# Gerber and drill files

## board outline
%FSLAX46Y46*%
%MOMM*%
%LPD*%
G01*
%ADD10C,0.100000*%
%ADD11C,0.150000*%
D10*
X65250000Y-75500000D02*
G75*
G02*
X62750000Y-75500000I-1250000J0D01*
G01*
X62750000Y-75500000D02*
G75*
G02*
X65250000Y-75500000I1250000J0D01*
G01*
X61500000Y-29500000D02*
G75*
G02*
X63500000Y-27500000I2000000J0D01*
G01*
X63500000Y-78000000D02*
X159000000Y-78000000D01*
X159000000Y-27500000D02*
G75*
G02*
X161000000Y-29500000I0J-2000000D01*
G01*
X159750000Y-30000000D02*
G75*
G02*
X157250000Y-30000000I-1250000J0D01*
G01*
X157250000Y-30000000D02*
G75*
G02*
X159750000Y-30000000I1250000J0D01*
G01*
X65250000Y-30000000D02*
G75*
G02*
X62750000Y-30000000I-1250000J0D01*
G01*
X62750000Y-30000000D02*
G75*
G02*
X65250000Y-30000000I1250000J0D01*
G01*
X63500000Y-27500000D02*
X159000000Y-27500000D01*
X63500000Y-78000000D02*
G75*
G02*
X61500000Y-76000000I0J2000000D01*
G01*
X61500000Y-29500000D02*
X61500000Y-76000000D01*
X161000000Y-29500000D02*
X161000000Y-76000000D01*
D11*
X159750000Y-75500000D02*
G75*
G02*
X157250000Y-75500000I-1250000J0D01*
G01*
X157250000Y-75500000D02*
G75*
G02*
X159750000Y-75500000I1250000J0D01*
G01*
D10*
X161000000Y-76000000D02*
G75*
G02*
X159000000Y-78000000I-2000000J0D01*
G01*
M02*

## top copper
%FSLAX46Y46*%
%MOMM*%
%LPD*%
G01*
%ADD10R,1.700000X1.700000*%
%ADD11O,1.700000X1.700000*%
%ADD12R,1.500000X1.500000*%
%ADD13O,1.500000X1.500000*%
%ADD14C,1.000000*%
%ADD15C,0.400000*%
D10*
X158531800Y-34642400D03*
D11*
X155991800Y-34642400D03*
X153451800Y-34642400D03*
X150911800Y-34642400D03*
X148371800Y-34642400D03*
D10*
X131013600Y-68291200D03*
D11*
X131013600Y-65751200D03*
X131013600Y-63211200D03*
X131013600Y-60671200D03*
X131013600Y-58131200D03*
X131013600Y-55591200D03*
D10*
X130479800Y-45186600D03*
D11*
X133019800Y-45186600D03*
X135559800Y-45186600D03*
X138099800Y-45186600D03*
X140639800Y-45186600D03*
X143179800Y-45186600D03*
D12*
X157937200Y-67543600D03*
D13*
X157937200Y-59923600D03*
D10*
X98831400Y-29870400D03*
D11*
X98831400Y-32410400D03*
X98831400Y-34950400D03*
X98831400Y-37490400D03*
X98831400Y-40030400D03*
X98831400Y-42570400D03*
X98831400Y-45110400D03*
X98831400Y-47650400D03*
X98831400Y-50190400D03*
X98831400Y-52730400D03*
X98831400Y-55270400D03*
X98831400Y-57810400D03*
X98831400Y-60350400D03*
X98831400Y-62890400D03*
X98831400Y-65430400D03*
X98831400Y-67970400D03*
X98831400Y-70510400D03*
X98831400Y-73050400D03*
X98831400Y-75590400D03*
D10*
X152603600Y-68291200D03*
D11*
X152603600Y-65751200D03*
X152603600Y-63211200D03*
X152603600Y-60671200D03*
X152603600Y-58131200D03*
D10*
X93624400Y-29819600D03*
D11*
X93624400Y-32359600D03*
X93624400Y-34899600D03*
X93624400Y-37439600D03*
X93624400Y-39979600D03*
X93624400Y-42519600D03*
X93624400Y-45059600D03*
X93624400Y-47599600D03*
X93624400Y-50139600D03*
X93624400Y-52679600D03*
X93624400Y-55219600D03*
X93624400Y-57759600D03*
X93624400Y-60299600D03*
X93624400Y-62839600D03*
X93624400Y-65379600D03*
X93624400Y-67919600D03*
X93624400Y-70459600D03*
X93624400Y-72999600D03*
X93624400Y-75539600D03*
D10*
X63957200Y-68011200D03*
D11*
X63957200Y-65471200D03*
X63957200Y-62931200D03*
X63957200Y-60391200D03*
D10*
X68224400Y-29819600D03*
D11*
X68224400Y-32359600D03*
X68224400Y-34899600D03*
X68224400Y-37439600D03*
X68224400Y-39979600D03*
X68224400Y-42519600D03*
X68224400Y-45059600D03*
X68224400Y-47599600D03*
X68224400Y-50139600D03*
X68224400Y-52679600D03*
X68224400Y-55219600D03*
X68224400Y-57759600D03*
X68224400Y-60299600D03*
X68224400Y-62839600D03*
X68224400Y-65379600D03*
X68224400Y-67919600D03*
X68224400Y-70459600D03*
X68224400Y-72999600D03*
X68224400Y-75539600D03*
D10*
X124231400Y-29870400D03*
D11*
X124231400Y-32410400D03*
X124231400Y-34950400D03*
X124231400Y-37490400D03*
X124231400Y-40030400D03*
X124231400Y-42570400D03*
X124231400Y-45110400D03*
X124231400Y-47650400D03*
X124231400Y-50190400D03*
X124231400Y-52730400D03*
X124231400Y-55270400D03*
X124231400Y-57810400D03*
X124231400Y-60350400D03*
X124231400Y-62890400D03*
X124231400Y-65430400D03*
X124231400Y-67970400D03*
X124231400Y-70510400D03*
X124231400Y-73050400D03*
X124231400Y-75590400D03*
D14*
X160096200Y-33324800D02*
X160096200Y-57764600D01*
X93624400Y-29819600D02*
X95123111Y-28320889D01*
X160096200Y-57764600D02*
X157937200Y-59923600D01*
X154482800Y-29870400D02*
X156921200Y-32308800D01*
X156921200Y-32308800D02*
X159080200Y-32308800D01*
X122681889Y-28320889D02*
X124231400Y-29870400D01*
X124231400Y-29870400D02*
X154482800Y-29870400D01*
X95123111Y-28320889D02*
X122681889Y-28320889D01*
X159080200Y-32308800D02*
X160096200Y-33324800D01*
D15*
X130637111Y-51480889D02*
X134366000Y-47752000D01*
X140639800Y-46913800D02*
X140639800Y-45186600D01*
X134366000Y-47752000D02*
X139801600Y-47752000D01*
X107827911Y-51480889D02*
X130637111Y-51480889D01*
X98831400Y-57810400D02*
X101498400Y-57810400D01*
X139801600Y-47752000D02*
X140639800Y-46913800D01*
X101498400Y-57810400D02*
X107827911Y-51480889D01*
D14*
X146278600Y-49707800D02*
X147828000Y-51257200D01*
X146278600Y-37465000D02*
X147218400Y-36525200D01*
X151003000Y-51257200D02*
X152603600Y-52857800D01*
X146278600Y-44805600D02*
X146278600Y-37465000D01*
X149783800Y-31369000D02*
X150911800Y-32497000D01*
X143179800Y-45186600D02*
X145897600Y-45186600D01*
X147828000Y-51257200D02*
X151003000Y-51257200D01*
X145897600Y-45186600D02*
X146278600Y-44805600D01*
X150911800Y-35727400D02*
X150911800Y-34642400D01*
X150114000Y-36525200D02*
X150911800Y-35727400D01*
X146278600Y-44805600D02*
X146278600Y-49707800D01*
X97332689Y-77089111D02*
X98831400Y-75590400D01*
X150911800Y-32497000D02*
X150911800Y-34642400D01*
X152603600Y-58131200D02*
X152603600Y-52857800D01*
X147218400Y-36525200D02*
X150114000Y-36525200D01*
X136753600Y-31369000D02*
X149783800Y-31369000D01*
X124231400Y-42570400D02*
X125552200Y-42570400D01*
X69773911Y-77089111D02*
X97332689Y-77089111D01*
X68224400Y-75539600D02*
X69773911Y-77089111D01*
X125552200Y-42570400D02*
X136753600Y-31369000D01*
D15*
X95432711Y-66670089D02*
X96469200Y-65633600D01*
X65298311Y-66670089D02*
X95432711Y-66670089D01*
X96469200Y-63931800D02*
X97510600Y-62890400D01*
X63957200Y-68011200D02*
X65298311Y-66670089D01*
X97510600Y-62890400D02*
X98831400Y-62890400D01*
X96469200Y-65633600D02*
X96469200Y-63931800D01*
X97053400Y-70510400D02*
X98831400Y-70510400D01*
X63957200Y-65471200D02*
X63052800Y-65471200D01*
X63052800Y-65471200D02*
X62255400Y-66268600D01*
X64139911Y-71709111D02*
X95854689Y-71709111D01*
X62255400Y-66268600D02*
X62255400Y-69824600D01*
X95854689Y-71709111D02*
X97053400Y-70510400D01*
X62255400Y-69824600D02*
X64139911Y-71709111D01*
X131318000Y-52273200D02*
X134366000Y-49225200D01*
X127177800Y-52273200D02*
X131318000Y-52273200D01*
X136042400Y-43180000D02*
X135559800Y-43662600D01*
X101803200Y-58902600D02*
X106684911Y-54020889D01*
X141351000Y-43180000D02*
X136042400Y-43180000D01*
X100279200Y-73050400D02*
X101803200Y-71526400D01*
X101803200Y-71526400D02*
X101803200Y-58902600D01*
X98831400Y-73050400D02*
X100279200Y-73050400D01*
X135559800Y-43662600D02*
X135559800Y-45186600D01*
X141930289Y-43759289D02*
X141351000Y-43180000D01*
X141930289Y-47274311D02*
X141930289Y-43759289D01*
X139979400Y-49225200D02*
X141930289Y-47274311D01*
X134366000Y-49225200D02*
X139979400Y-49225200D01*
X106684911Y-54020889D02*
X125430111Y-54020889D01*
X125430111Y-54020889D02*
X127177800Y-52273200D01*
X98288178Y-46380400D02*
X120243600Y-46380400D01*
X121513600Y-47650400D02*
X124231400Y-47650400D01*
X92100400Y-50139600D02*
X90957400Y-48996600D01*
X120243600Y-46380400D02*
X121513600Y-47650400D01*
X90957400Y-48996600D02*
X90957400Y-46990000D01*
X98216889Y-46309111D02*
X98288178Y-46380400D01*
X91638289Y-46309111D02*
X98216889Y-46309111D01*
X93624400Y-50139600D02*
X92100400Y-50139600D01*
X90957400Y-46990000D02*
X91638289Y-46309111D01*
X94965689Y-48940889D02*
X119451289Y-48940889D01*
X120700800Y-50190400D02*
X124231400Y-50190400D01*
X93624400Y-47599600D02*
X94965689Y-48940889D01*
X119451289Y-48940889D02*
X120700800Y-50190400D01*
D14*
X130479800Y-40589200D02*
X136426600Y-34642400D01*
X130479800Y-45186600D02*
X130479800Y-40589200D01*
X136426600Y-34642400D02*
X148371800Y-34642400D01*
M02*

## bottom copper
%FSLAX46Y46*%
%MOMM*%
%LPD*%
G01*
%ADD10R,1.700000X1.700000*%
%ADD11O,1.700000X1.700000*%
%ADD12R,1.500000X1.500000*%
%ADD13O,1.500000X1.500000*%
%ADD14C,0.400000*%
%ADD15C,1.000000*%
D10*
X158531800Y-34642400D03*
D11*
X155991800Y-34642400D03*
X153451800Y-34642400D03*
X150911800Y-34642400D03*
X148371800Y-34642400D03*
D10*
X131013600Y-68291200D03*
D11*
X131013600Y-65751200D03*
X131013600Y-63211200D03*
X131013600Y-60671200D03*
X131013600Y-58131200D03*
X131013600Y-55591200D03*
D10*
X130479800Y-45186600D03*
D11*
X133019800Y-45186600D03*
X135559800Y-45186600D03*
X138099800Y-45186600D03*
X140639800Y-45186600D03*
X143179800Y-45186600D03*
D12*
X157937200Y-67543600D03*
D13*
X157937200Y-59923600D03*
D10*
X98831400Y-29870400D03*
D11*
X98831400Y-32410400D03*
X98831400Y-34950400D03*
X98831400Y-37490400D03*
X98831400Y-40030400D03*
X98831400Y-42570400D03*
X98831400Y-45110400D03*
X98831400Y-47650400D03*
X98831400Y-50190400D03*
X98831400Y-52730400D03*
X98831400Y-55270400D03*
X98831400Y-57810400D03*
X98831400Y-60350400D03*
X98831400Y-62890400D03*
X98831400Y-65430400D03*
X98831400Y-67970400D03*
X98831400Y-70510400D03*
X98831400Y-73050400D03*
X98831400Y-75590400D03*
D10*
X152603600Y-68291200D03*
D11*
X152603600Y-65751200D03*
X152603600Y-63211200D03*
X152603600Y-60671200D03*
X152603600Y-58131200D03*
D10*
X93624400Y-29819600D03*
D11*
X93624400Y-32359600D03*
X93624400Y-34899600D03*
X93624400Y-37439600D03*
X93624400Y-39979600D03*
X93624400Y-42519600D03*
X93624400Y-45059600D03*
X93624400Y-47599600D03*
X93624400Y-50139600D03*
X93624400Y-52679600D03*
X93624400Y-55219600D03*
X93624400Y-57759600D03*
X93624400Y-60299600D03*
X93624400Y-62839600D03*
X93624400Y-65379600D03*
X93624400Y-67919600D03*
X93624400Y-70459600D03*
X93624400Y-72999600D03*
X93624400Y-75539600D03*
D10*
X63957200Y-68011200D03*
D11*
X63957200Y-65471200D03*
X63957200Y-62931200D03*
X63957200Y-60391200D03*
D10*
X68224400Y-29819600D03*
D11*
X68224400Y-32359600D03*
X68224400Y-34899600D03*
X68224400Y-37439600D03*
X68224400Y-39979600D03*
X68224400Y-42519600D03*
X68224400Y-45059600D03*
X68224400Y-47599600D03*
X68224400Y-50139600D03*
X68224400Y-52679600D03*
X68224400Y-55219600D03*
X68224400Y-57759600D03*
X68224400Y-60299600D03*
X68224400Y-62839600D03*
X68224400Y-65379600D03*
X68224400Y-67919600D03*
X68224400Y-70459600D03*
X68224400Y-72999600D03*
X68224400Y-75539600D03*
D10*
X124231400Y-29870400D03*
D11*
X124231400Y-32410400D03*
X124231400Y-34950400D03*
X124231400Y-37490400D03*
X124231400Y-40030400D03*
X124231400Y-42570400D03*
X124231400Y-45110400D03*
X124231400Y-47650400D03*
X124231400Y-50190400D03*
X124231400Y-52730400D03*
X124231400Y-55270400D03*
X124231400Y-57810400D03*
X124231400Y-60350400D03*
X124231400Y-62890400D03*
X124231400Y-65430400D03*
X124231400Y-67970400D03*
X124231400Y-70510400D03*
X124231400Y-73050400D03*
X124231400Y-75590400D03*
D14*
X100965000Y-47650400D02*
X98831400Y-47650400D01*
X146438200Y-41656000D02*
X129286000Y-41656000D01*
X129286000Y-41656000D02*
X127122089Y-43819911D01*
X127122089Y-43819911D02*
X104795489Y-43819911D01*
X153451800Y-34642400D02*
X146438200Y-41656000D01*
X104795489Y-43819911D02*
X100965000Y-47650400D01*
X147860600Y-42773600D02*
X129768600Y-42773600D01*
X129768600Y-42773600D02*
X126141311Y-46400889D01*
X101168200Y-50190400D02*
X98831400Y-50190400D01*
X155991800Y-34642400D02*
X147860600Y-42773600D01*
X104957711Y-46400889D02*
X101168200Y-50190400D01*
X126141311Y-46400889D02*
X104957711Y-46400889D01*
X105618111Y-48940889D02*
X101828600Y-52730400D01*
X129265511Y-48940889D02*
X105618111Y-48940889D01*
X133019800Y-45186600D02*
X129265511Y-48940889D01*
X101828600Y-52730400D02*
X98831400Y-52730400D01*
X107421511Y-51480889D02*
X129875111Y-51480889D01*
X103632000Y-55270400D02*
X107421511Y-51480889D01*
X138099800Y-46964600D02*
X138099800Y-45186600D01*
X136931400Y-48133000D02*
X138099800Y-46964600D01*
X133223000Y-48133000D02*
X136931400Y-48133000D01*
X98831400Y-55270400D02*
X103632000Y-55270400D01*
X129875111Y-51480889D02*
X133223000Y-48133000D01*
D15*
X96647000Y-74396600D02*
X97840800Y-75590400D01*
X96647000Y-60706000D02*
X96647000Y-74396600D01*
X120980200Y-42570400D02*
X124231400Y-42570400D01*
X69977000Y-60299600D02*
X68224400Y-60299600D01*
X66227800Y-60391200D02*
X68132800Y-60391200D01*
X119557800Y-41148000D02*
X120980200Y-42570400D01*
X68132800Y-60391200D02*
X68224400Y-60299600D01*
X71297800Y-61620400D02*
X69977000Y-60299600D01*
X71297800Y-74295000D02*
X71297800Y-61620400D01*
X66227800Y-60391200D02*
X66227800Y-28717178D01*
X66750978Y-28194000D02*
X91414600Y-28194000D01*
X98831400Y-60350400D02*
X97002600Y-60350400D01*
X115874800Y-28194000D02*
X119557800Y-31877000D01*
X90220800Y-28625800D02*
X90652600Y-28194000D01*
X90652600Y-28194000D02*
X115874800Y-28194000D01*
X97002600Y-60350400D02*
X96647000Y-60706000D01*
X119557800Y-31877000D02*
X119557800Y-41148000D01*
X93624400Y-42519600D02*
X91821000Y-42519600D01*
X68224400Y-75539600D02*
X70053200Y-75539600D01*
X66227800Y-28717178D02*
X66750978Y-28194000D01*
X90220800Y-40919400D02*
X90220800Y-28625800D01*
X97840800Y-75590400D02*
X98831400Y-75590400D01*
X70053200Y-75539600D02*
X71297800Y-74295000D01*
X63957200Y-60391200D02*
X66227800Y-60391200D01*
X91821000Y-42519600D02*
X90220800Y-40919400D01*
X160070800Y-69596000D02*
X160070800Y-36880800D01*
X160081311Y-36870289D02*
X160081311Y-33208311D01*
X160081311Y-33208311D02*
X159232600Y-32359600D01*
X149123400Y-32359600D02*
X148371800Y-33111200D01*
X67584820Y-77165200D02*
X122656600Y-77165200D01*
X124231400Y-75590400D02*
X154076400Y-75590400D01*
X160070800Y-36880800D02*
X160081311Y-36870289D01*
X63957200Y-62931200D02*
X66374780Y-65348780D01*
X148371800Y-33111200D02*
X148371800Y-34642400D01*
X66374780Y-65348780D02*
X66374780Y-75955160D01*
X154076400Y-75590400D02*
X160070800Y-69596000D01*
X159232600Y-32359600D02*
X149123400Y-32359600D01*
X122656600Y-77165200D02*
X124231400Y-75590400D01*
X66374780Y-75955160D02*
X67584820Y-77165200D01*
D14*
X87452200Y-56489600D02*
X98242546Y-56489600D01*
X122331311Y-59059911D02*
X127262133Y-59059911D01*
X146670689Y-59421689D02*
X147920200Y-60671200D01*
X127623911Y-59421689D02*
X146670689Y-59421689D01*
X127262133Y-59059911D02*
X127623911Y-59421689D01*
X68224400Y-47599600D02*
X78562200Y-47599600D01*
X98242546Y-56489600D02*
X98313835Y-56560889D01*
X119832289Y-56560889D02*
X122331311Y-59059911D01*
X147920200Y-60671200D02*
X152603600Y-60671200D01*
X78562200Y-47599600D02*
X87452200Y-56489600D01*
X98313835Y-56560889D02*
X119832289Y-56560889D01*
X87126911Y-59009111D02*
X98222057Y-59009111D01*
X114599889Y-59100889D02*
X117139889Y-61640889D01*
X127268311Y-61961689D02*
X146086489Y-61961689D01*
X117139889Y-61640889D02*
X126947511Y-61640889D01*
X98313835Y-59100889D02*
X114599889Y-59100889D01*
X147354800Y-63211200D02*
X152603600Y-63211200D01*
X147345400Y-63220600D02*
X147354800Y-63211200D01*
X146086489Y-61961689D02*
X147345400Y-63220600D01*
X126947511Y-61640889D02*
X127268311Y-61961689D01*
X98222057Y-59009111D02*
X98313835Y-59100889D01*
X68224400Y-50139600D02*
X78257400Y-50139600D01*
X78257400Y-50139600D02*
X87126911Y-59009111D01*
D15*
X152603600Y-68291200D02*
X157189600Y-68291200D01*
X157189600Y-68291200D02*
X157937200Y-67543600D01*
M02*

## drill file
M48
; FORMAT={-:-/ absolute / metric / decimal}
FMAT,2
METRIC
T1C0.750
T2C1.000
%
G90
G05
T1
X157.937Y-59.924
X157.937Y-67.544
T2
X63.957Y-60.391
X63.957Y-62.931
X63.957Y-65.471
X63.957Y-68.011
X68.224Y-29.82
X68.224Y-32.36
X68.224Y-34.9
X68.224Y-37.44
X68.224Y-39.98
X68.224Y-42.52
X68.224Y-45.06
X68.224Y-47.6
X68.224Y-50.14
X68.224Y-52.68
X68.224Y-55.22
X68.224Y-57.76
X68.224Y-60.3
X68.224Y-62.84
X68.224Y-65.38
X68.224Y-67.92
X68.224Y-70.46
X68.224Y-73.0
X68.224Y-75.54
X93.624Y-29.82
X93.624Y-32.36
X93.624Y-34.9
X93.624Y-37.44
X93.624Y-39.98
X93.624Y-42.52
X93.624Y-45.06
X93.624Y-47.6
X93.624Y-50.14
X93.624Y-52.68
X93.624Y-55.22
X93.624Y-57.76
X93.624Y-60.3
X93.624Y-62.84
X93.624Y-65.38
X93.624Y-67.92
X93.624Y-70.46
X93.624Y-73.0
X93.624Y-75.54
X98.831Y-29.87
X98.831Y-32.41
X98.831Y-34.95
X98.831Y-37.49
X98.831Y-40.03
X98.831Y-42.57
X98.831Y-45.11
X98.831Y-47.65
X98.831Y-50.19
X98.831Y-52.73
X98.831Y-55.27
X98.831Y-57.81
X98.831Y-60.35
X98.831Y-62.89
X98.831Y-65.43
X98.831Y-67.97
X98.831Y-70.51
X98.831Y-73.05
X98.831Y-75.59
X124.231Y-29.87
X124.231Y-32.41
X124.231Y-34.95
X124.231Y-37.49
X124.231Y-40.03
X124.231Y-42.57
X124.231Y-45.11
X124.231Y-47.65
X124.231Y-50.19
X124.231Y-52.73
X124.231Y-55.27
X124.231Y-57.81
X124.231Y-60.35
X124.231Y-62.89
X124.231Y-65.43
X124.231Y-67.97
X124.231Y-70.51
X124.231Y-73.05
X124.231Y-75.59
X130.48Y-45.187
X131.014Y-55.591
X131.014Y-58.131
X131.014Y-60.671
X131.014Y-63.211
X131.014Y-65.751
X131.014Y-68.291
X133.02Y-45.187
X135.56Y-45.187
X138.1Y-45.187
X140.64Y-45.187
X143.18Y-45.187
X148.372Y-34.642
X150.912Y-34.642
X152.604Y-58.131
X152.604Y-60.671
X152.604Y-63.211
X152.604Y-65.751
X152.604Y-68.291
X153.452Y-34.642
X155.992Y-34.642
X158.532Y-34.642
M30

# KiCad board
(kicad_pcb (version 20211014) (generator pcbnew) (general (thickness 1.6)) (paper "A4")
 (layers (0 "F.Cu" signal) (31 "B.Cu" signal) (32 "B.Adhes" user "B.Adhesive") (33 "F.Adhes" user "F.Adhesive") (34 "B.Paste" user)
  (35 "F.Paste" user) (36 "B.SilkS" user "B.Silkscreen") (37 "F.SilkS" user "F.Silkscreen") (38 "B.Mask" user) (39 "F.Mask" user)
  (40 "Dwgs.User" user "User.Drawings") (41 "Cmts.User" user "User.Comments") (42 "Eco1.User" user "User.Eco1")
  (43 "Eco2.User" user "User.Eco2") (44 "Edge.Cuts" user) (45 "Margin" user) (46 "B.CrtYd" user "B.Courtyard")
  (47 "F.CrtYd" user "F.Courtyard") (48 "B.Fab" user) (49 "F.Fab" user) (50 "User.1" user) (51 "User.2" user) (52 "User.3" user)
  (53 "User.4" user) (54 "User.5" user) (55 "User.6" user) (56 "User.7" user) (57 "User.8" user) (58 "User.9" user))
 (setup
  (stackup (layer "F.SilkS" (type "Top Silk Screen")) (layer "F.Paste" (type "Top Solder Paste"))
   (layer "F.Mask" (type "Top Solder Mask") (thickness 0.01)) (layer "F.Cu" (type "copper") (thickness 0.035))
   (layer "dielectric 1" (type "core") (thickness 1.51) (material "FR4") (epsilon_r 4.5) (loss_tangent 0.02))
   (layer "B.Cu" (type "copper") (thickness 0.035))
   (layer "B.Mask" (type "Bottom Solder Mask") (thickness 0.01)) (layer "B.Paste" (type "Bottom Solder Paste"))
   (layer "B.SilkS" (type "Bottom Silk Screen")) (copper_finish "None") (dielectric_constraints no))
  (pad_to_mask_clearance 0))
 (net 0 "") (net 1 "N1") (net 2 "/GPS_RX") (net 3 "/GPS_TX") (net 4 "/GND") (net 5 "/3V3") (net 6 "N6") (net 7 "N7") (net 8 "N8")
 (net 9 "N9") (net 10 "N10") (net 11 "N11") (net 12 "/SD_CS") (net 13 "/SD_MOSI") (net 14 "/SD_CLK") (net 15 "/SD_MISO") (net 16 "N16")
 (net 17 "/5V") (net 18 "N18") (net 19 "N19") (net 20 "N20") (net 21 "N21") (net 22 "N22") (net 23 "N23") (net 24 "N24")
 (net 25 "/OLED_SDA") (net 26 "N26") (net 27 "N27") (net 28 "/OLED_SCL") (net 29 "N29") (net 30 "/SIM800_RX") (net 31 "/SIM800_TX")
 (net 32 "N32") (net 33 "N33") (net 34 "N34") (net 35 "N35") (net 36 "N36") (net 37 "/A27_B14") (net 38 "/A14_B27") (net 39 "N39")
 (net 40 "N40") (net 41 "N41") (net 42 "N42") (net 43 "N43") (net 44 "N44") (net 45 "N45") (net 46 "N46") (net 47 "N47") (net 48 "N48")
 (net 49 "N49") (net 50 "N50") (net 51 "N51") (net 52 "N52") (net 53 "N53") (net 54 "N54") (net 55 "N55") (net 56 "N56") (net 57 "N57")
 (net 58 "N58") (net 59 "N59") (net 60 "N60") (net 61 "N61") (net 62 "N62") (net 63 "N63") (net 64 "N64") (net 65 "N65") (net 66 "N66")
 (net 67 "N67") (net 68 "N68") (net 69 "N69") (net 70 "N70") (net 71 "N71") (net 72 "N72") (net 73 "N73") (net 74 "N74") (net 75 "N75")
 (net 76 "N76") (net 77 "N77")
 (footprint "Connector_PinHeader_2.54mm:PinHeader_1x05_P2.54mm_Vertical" (layer "F.Cu") (at 158.5318 34.6424 -90)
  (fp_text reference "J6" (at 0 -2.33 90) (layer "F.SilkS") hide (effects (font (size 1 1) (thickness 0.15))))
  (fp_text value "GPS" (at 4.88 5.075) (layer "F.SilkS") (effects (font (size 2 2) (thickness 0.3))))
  (pad "1" thru_hole rect (at 0 0 270) (size 1.7 1.7) (drill 1) (layers *.Cu *.Mask) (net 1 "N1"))
  (pad "2" thru_hole oval (at 0 2.54 270) (size 1.7 1.7) (drill 1) (layers *.Cu *.Mask) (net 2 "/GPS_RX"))
  (pad "3" thru_hole oval (at 0 5.08 270) (size 1.7 1.7) (drill 1) (layers *.Cu *.Mask) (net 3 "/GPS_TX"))
  (pad "4" thru_hole oval (at 0 7.62 270) (size 1.7 1.7) (drill 1) (layers *.Cu *.Mask) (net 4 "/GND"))
  (pad "5" thru_hole oval (at 0 10.16 270) (size 1.7 1.7) (drill 1) (layers *.Cu *.Mask) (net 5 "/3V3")))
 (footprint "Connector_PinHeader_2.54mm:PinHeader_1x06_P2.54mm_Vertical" (layer "F.Cu") (at 131.0136 68.2912 180)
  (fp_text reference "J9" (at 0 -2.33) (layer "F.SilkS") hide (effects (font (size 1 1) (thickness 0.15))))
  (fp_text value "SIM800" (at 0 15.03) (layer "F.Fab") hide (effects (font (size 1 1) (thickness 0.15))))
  (pad "1" thru_hole rect (at 0 0 180) (size 1.7 1.7) (drill 1) (layers *.Cu *.Mask) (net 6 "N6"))
  (pad "2" thru_hole oval (at 0 2.54 180) (size 1.7 1.7) (drill 1) (layers *.Cu *.Mask) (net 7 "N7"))
  (pad "3" thru_hole oval (at 0 5.08 180) (size 1.7 1.7) (drill 1) (layers *.Cu *.Mask) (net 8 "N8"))
  (pad "4" thru_hole oval (at 0 7.62 180) (size 1.7 1.7) (drill 1) (layers *.Cu *.Mask) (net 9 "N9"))
  (pad "5" thru_hole oval (at 0 10.16 180) (size 1.7 1.7) (drill 1) (layers *.Cu *.Mask) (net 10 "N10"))
  (pad "6" thru_hole oval (at 0 12.7 180) (size 1.7 1.7) (drill 1) (layers *.Cu *.Mask) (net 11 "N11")))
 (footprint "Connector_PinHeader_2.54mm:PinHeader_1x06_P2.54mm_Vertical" (layer "F.Cu") (at 130.4798 45.1866 90)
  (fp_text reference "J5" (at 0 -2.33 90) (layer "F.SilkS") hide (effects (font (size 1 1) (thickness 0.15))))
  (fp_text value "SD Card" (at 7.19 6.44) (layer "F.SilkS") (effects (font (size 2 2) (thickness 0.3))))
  (pad "1" thru_hole rect (at 0 0 90) (size 1.7 1.7) (drill 1) (layers *.Cu *.Mask) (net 5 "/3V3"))
  (pad "2" thru_hole oval (at 0 2.54 90) (size 1.7 1.7) (drill 1) (layers *.Cu *.Mask) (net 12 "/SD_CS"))
  (pad "3" thru_hole oval (at 0 5.08 90) (size 1.7 1.7) (drill 1) (layers *.Cu *.Mask) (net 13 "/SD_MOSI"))
  (pad "4" thru_hole oval (at 0 7.62 90) (size 1.7 1.7) (drill 1) (layers *.Cu *.Mask) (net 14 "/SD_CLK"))
  (pad "5" thru_hole oval (at 0 10.16 90) (size 1.7 1.7) (drill 1) (layers *.Cu *.Mask) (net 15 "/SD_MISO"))
  (pad "6" thru_hole oval (at 0 12.7 90) (size 1.7 1.7) (drill 1) (layers *.Cu *.Mask) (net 4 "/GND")))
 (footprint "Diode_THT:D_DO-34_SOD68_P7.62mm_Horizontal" (layer "F.Cu") (at 157.9372 67.5436 90)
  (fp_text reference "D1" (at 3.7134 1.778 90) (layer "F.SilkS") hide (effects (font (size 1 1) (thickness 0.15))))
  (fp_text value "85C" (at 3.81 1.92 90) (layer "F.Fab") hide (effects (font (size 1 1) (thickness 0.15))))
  (pad "1" thru_hole rect (at 0 0 90) (size 1.5 1.5) (drill 0.75) (layers *.Cu *.Mask) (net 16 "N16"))
  (pad "2" thru_hole oval (at 7.62 0 90) (size 1.5 1.5) (drill 0.75) (layers *.Cu *.Mask) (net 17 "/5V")))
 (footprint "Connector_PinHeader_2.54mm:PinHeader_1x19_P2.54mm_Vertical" (layer "F.Cu") (at 98.8314 29.8704)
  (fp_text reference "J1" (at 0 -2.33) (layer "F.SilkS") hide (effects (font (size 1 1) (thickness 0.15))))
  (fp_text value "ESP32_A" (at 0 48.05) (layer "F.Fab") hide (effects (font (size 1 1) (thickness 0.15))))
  (pad "1" thru_hole rect (at 0 0) (size 1.7 1.7) (drill 1) (layers *.Cu *.Mask) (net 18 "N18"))
  (pad "2" thru_hole oval (at 0 2.54) (size 1.7 1.7) (drill 1) (layers *.Cu *.Mask) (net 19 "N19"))
  (pad "3" thru_hole oval (at 0 5.08) (size 1.7 1.7) (drill 1) (layers *.Cu *.Mask) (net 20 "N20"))
  (pad "4" thru_hole oval (at 0 7.62) (size 1.7 1.7) (drill 1) (layers *.Cu *.Mask) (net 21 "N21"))
  (pad "5" thru_hole oval (at 0 10.16) (size 1.7 1.7) (drill 1) (layers *.Cu *.Mask) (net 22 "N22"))
  (pad "6" thru_hole oval (at 0 12.7) (size 1.7 1.7) (drill 1) (layers *.Cu *.Mask) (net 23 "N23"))
  (pad "7" thru_hole oval (at 0 15.24) (size 1.7 1.7) (drill 1) (layers *.Cu *.Mask) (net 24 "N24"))
  (pad "8" thru_hole oval (at 0 17.78) (size 1.7 1.7) (drill 1) (layers *.Cu *.Mask) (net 3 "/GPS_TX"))
  (pad "9" thru_hole oval (at 0 20.32) (size 1.7 1.7) (drill 1) (layers *.Cu *.Mask) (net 2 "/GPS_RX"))
  (pad "10" thru_hole oval (at 0 22.86) (size 1.7 1.7) (drill 1) (layers *.Cu *.Mask) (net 12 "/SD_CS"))
  (pad "11" thru_hole oval (at 0 25.4) (size 1.7 1.7) (drill 1) (layers *.Cu *.Mask) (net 14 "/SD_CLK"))
  (pad "12" thru_hole oval (at 0 27.94) (size 1.7 1.7) (drill 1) (layers *.Cu *.Mask) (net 15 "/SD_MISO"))
  (pad "13" thru_hole oval (at 0 30.48) (size 1.7 1.7) (drill 1) (layers *.Cu *.Mask) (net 4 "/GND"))
  (pad "14" thru_hole oval (at 0 33.02) (size 1.7 1.7) (drill 1) (layers *.Cu *.Mask) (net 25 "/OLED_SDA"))
  (pad "15" thru_hole oval (at 0 35.56) (size 1.7 1.7) (drill 1) (layers *.Cu *.Mask) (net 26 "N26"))
  (pad "16" thru_hole oval (at 0 38.1) (size 1.7 1.7) (drill 1) (layers *.Cu *.Mask) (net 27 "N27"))
  (pad "17" thru_hole oval (at 0 40.64) (size 1.7 1.7) (drill 1) (layers *.Cu *.Mask) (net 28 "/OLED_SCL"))
  (pad "18" thru_hole oval (at 0 43.18) (size 1.7 1.7) (drill 1) (layers *.Cu *.Mask) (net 13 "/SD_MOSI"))
  (pad "19" thru_hole oval (at 0 45.72) (size 1.7 1.7) (drill 1) (layers *.Cu *.Mask) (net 4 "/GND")))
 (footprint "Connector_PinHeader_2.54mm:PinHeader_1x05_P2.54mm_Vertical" (layer "F.Cu") (at 152.6036 68.2912 180)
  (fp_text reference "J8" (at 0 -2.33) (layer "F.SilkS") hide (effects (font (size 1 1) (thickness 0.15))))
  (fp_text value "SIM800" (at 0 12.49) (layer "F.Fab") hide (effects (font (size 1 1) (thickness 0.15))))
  (pad "1" thru_hole rect (at 0 0 180) (size 1.7 1.7) (drill 1) (layers *.Cu *.Mask) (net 16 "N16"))
  (pad "2" thru_hole oval (at 0 2.54 180) (size 1.7 1.7) (drill 1) (layers *.Cu *.Mask) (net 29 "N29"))
  (pad "3" thru_hole oval (at 0 5.08 180) (size 1.7 1.7) (drill 1) (layers *.Cu *.Mask) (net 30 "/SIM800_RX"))
  (pad "4" thru_hole oval (at 0 7.62 180) (size 1.7 1.7) (drill 1) (layers *.Cu *.Mask) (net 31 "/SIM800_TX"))
  (pad "5" thru_hole oval (at 0 10.16 180) (size 1.7 1.7) (drill 1) (layers *.Cu *.Mask) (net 4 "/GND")))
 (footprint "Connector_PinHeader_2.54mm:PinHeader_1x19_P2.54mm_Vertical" (layer "F.Cu") (at 93.6244 29.8196)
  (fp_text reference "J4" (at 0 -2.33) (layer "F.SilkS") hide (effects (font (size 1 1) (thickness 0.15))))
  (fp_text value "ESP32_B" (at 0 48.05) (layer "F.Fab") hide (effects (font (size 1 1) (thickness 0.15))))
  (pad "1" thru_hole rect (at 0 0) (size 1.7 1.7) (drill 1) (layers *.Cu *.Mask) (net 17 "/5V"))
  (pad "2" thru_hole oval (at 0 2.54) (size 1.7 1.7) (drill 1) (layers *.Cu *.Mask) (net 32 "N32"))
  (pad "3" thru_hole oval (at 0 5.08) (size 1.7 1.7) (drill 1) (layers *.Cu *.Mask) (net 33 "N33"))
  (pad "4" thru_hole oval (at 0 7.62) (size 1.7 1.7) (drill 1) (layers *.Cu *.Mask) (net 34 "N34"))
  (pad "5" thru_hole oval (at 0 10.16) (size 1.7 1.7) (drill 1) (layers *.Cu *.Mask) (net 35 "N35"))
  (pad "6" thru_hole oval (at 0 12.7) (size 1.7 1.7) (drill 1) (layers *.Cu *.Mask) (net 4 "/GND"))
  (pad "7" thru_hole oval (at 0 15.24) (size 1.7 1.7) (drill 1) (layers *.Cu *.Mask) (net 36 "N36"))
  (pad "8" thru_hole oval (at 0 17.78) (size 1.7 1.7) (drill 1) (layers *.Cu *.Mask) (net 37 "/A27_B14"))
  (pad "9" thru_hole oval (at 0 20.32) (size 1.7 1.7) (drill 1) (layers *.Cu *.Mask) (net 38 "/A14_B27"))
  (pad "10" thru_hole oval (at 0 22.86) (size 1.7 1.7) (drill 1) (layers *.Cu *.Mask) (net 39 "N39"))
  (pad "11" thru_hole oval (at 0 25.4) (size 1.7 1.7) (drill 1) (layers *.Cu *.Mask) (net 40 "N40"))
  (pad "12" thru_hole oval (at 0 27.94) (size 1.7 1.7) (drill 1) (layers *.Cu *.Mask) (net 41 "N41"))
  (pad "13" thru_hole oval (at 0 30.48) (size 1.7 1.7) (drill 1) (layers *.Cu *.Mask) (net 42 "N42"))
  (pad "14" thru_hole oval (at 0 33.02) (size 1.7 1.7) (drill 1) (layers *.Cu *.Mask) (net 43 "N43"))
  (pad "15" thru_hole oval (at 0 35.56) (size 1.7 1.7) (drill 1) (layers *.Cu *.Mask) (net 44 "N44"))
  (pad "16" thru_hole oval (at 0 38.1) (size 1.7 1.7) (drill 1) (layers *.Cu *.Mask) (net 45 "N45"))
  (pad "17" thru_hole oval (at 0 40.64) (size 1.7 1.7) (drill 1) (layers *.Cu *.Mask) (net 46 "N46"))
  (pad "18" thru_hole oval (at 0 43.18) (size 1.7 1.7) (drill 1) (layers *.Cu *.Mask) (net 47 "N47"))
  (pad "19" thru_hole oval (at 0 45.72) (size 1.7 1.7) (drill 1) (layers *.Cu *.Mask) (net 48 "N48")))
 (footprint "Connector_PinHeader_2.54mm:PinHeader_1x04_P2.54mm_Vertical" (layer "F.Cu") (at 63.9572 68.0112 180)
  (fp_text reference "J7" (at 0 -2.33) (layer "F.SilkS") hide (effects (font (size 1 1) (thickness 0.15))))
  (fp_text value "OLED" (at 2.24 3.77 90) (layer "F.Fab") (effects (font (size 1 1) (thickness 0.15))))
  (pad "1" thru_hole rect (at 0 0 180) (size 1.7 1.7) (drill 1) (layers *.Cu *.Mask) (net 25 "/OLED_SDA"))
  (pad "2" thru_hole oval (at 0 2.54 180) (size 1.7 1.7) (drill 1) (layers *.Cu *.Mask) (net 28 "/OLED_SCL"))
  (pad "3" thru_hole oval (at 0 5.08 180) (size 1.7 1.7) (drill 1) (layers *.Cu *.Mask) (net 5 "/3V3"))
  (pad "4" thru_hole oval (at 0 7.62 180) (size 1.7 1.7) (drill 1) (layers *.Cu *.Mask) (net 4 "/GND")))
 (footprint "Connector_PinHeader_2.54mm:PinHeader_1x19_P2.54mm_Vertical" (layer "F.Cu") (at 68.2244 29.8196)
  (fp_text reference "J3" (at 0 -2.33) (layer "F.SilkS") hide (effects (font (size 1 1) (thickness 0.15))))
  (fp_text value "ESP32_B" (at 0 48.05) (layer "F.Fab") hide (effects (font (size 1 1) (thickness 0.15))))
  (pad "1" thru_hole rect (at 0 0) (size 1.7 1.7) (drill 1) (layers *.Cu *.Mask) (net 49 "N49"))
  (pad "2" thru_hole oval (at 0 2.54) (size 1.7 1.7) (drill 1) (layers *.Cu *.Mask) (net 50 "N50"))
  (pad "3" thru_hole oval (at 0 5.08) (size 1.7 1.7) (drill 1) (layers *.Cu *.Mask) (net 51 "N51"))
  (pad "4" thru_hole oval (at 0 7.62) (size 1.7 1.7) (drill 1) (layers *.Cu *.Mask) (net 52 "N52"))
  (pad "5" thru_hole oval (at 0 10.16) (size 1.7 1.7) (drill 1) (layers *.Cu *.Mask) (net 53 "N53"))
  (pad "6" thru_hole oval (at 0 12.7) (size 1.7 1.7) (drill 1) (layers *.Cu *.Mask) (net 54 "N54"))
  (pad "7" thru_hole oval (at 0 15.24) (size 1.7 1.7) (drill 1) (layers *.Cu *.Mask) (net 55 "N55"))
  (pad "8" thru_hole oval (at 0 17.78) (size 1.7 1.7) (drill 1) (layers *.Cu *.Mask) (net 31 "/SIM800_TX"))
  (pad "9" thru_hole oval (at 0 20.32) (size 1.7 1.7) (drill 1) (layers *.Cu *.Mask) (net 30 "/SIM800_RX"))
  (pad "10" thru_hole oval (at 0 22.86) (size 1.7 1.7) (drill 1) (layers *.Cu *.Mask) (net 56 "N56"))
  (pad "11" thru_hole oval (at 0 25.4) (size 1.7 1.7) (drill 1) (layers *.Cu *.Mask) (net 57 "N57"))
  (pad "12" thru_hole oval (at 0 27.94) (size 1.7 1.7) (drill 1) (layers *.Cu *.Mask) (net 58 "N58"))
  (pad "13" thru_hole oval (at 0 30.48) (size 1.7 1.7) (drill 1) (layers *.Cu *.Mask) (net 4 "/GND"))
  (pad "14" thru_hole oval (at 0 33.02) (size 1.7 1.7) (drill 1) (layers *.Cu *.Mask) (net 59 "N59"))
  (pad "15" thru_hole oval (at 0 35.56) (size 1.7 1.7) (drill 1) (layers *.Cu *.Mask) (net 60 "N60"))
  (pad "16" thru_hole oval (at 0 38.1) (size 1.7 1.7) (drill 1) (layers *.Cu *.Mask) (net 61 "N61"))
  (pad "17" thru_hole oval (at 0 40.64) (size 1.7 1.7) (drill 1) (layers *.Cu *.Mask) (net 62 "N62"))
  (pad "18" thru_hole oval (at 0 43.18) (size 1.7 1.7) (drill 1) (layers *.Cu *.Mask) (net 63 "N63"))
  (pad "19" thru_hole oval (at 0 45.72) (size 1.7 1.7) (drill 1) (layers *.Cu *.Mask) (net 4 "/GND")))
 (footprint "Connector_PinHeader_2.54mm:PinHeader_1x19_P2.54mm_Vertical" (layer "F.Cu") (at 124.2314 29.8704)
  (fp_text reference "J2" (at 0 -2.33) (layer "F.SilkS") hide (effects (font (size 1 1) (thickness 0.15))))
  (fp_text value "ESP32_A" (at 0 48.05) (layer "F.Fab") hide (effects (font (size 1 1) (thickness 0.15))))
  (pad "1" thru_hole rect (at 0 0) (size 1.7 1.7) (drill 1) (layers *.Cu *.Mask) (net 17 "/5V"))
  (pad "2" thru_hole oval (at 0 2.54) (size 1.7 1.7) (drill 1) (layers *.Cu *.Mask) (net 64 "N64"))
  (pad "3" thru_hole oval (at 0 5.08) (size 1.7 1.7) (drill 1) (layers *.Cu *.Mask) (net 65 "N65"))
  (pad "4" thru_hole oval (at 0 7.62) (size 1.7 1.7) (drill 1) (layers *.Cu *.Mask) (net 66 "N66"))
  (pad "5" thru_hole oval (at 0 10.16) (size 1.7 1.7) (drill 1) (layers *.Cu *.Mask) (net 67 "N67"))
  (pad "6" thru_hole oval (at 0 12.7) (size 1.7 1.7) (drill 1) (layers *.Cu *.Mask) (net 4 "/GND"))
  (pad "7" thru_hole oval (at 0 15.24) (size 1.7 1.7) (drill 1) (layers *.Cu *.Mask) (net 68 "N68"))
  (pad "8" thru_hole oval (at 0 17.78) (size 1.7 1.7) (drill 1) (layers *.Cu *.Mask) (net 38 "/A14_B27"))
  (pad "9" thru_hole oval (at 0 20.32) (size 1.7 1.7) (drill 1) (layers *.Cu *.Mask) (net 37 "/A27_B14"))
  (pad "10" thru_hole oval (at 0 22.86) (size 1.7 1.7) (drill 1) (layers *.Cu *.Mask) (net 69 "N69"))
  (pad "11" thru_hole oval (at 0 25.4) (size 1.7 1.7) (drill 1) (layers *.Cu *.Mask) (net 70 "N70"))
  (pad "12" thru_hole oval (at 0 27.94) (size 1.7 1.7) (drill 1) (layers *.Cu *.Mask) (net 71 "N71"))
  (pad "13" thru_hole oval (at 0 30.48) (size 1.7 1.7) (drill 1) (layers *.Cu *.Mask) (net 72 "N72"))
  (pad "14" thru_hole oval (at 0 33.02) (size 1.7 1.7) (drill 1) (layers *.Cu *.Mask) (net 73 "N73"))
  (pad "15" thru_hole oval (at 0 35.56) (size 1.7 1.7) (drill 1) (layers *.Cu *.Mask) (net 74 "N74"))
  (pad "16" thru_hole oval (at 0 38.1) (size 1.7 1.7) (drill 1) (layers *.Cu *.Mask) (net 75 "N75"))
  (pad "17" thru_hole oval (at 0 40.64) (size 1.7 1.7) (drill 1) (layers *.Cu *.Mask) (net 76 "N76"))
  (pad "18" thru_hole oval (at 0 43.18) (size 1.7 1.7) (drill 1) (layers *.Cu *.Mask) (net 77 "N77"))
  (pad "19" thru_hole oval (at 0 45.72) (size 1.7 1.7) (drill 1) (layers *.Cu *.Mask) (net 5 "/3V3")))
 (gr_circle (center 64 75.5) (end 65.25 75.5) (layer "Edge.Cuts") (width 0.1) (fill none))
 (gr_arc (start 61.5 29.5) (mid 62.085786 28.085786) (end 63.5 27.5) (layer "Edge.Cuts") (width 0.1))
 (gr_line (start 63.5 78) (end 159 78) (layer "Edge.Cuts") (width 0.1))
 (gr_arc (start 159 27.5) (mid 160.414214 28.085786) (end 161 29.5) (layer "Edge.Cuts") (width 0.1))
 (gr_circle (center 158.5 30) (end 159.75 30) (layer "Edge.Cuts") (width 0.1) (fill none))
 (gr_circle (center 64 30) (end 65.25 30) (layer "Edge.Cuts") (width 0.1) (fill none))
 (gr_line (start 63.5 27.5) (end 159 27.5) (layer "Edge.Cuts") (width 0.1))
 (gr_arc (start 63.5 78) (mid 62.085786 77.414214) (end 61.5 76) (layer "Edge.Cuts") (width 0.1))
 (gr_line (start 61.5 29.5) (end 61.5 76) (layer "Edge.Cuts") (width 0.1))
 (gr_line (start 161 29.5) (end 161 76) (layer "Edge.Cuts") (width 0.1))
 (gr_circle (center 158.5 75.5) (end 159.75 75.5) (layer "Edge.Cuts") (width 0.15) (fill none))
 (gr_arc (start 161 76) (mid 160.414214 77.414214) (end 159 78) (layer "Edge.Cuts") (width 0.1))
 (segment (start 160.0962 33.3248) (end 160.0962 57.7646) (width 1) (layer "F.Cu") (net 17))
 (segment (start 93.6244 29.8196) (end 95.123111 28.320889) (width 1) (layer "F.Cu") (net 17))
 (segment (start 160.0962 57.7646) (end 157.9372 59.9236) (width 1) (layer "F.Cu") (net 17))
 (segment (start 154.4828 29.8704) (end 156.9212 32.3088) (width 1) (layer "F.Cu") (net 17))
 (segment (start 156.9212 32.3088) (end 159.0802 32.3088) (width 1) (layer "F.Cu") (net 17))
 (segment (start 122.681889 28.320889) (end 124.2314 29.8704) (width 1) (layer "F.Cu") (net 17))
 (segment (start 124.2314 29.8704) (end 154.4828 29.8704) (width 1) (layer "F.Cu") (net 17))
 (segment (start 95.123111 28.320889) (end 122.681889 28.320889) (width 1) (layer "F.Cu") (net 17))
 (segment (start 159.0802 32.3088) (end 160.0962 33.3248) (width 1) (layer "F.Cu") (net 17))
 (segment (start 100.965 47.6504) (end 98.8314 47.6504) (width 0.4) (layer "B.Cu") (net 3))
 (segment (start 146.4382 41.656) (end 129.286 41.656) (width 0.4) (layer "B.Cu") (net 3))
 (segment (start 129.286 41.656) (end 127.122089 43.819911) (width 0.4) (layer "B.Cu") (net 3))
 (segment (start 127.122089 43.819911) (end 104.795489 43.819911) (width 0.4) (layer "B.Cu") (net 3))
 (segment (start 153.4518 34.6424) (end 146.4382 41.656) (width 0.4) (layer "B.Cu") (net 3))
 (segment (start 104.795489 43.819911) (end 100.965 47.6504) (width 0.4) (layer "B.Cu") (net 3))
 (segment (start 147.8606 42.7736) (end 129.7686 42.7736) (width 0.4) (layer "B.Cu") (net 2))
 (segment (start 129.7686 42.7736) (end 126.141311 46.400889) (width 0.4) (layer "B.Cu") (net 2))
 (segment (start 101.1682 50.1904) (end 98.8314 50.1904) (width 0.4) (layer "B.Cu") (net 2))
 (segment (start 155.9918 34.6424) (end 147.8606 42.7736) (width 0.4) (layer "B.Cu") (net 2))
 (segment (start 104.957711 46.400889) (end 101.1682 50.1904) (width 0.4) (layer "B.Cu") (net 2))
 (segment (start 126.141311 46.400889) (end 104.957711 46.400889) (width 0.4) (layer "B.Cu") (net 2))
 (segment (start 105.618111 48.940889) (end 101.8286 52.7304) (width 0.4) (layer "B.Cu") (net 12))
 (segment (start 129.265511 48.940889) (end 105.618111 48.940889) (width 0.4) (layer "B.Cu") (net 12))
 (segment (start 133.0198 45.1866) (end 129.265511 48.940889) (width 0.4) (layer "B.Cu") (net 12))
 (segment (start 101.8286 52.7304) (end 98.8314 52.7304) (width 0.4) (layer "B.Cu") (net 12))
 (segment (start 107.421511 51.480889) (end 129.875111 51.480889) (width 0.4) (layer "B.Cu") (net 14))
 (segment (start 103.632 55.2704) (end 107.421511 51.480889) (width 0.4) (layer "B.Cu") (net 14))
 (segment (start 138.0998 46.9646) (end 138.0998 45.1866) (width 0.4) (layer "B.Cu") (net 14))
 (segment (start 136.9314 48.133) (end 138.0998 46.9646) (width 0.4) (layer "B.Cu") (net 14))
 (segment (start 133.223 48.133) (end 136.9314 48.133) (width 0.4) (layer "B.Cu") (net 14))
 (segment (start 98.8314 55.2704) (end 103.632 55.2704) (width 0.4) (layer "B.Cu") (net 14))
 (segment (start 129.875111 51.480889) (end 133.223 48.133) (width 0.4) (layer "B.Cu") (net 14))
 (segment (start 130.637111 51.480889) (end 134.366 47.752) (width 0.4) (layer "F.Cu") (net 15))
 (segment (start 140.6398 46.9138) (end 140.6398 45.1866) (width 0.4) (layer "F.Cu") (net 15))
 (segment (start 134.366 47.752) (end 139.8016 47.752) (width 0.4) (layer "F.Cu") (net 15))
 (segment (start 107.827911 51.480889) (end 130.637111 51.480889) (width 0.4) (layer "F.Cu") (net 15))
 (segment (start 98.8314 57.8104) (end 101.4984 57.8104) (width 0.4) (layer "F.Cu") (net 15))
 (segment (start 139.8016 47.752) (end 140.6398 46.9138) (width 0.4) (layer "F.Cu") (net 15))
 (segment (start 101.4984 57.8104) (end 107.827911 51.480889) (width 0.4) (layer "F.Cu") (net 15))
 (segment (start 146.2786 49.7078) (end 147.828 51.2572) (width 1) (layer "F.Cu") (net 4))
 (segment (start 146.2786 37.465) (end 147.2184 36.5252) (width 1) (layer "F.Cu") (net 4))
 (segment (start 151.003 51.2572) (end 152.6036 52.8578) (width 1) (layer "F.Cu") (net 4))
 (segment (start 146.2786 44.8056) (end 146.2786 37.465) (width 1) (layer "F.Cu") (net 4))
 (segment (start 149.7838 31.369) (end 150.9118 32.497) (width 1) (layer "F.Cu") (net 4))
 (segment (start 143.1798 45.1866) (end 145.8976 45.1866) (width 1) (layer "F.Cu") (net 4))
 (segment (start 147.828 51.2572) (end 151.003 51.2572) (width 1) (layer "F.Cu") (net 4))
 (segment (start 145.8976 45.1866) (end 146.2786 44.8056) (width 1) (layer "F.Cu") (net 4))
 (segment (start 150.9118 35.7274) (end 150.9118 34.6424) (width 1) (layer "F.Cu") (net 4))
 (segment (start 150.114 36.5252) (end 150.9118 35.7274) (width 1) (layer "F.Cu") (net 4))
 (segment (start 146.2786 44.8056) (end 146.2786 49.7078) (width 1) (layer "F.Cu") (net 4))
 (segment (start 97.332689 77.089111) (end 98.8314 75.5904) (width 1) (layer "F.Cu") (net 4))
 (segment (start 150.9118 32.497) (end 150.9118 34.6424) (width 1) (layer "F.Cu") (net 4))
 (segment (start 152.6036 58.1312) (end 152.6036 52.8578) (width 1) (layer "F.Cu") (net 4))
 (segment (start 147.2184 36.5252) (end 150.114 36.5252) (width 1) (layer "F.Cu") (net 4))
 (segment (start 136.7536 31.369) (end 149.7838 31.369) (width 1) (layer "F.Cu") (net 4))
 (segment (start 124.2314 42.5704) (end 125.5522 42.5704) (width 1) (layer "F.Cu") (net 4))
 (segment (start 69.773911 77.089111) (end 97.332689 77.089111) (width 1) (layer "F.Cu") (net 4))
 (segment (start 68.2244 75.5396) (end 69.773911 77.089111) (width 1) (layer "F.Cu") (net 4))
 (segment (start 125.5522 42.5704) (end 136.7536 31.369) (width 1) (layer "F.Cu") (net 4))
 (segment (start 96.647 74.3966) (end 97.8408 75.5904) (width 1) (layer "B.Cu") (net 4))
 (segment (start 96.647 60.706) (end 96.647 74.3966) (width 1) (layer "B.Cu") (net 4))
 (segment (start 120.9802 42.5704) (end 124.2314 42.5704) (width 1) (layer "B.Cu") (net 4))
 (segment (start 69.977 60.2996) (end 68.2244 60.2996) (width 1) (layer "B.Cu") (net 4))
 (segment (start 66.2278 60.3912) (end 68.1328 60.3912) (width 1) (layer "B.Cu") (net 4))
 (segment (start 119.5578 41.148) (end 120.9802 42.5704) (width 1) (layer "B.Cu") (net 4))
 (segment (start 68.1328 60.3912) (end 68.2244 60.2996) (width 1) (layer "B.Cu") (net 4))
 (segment (start 71.2978 61.6204) (end 69.977 60.2996) (width 1) (layer "B.Cu") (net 4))
 (segment (start 71.2978 74.295) (end 71.2978 61.6204) (width 1) (layer "B.Cu") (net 4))
 (segment (start 66.2278 60.3912) (end 66.2278 28.717178) (width 1) (layer "B.Cu") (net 4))
 (segment (start 66.750978 28.194) (end 91.4146 28.194) (width 1) (layer "B.Cu") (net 4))
 (segment (start 98.8314 60.3504) (end 97.0026 60.3504) (width 1) (layer "B.Cu") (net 4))
 (segment (start 115.8748 28.194) (end 119.5578 31.877) (width 1) (layer "B.Cu") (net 4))
 (segment (start 90.2208 28.6258) (end 90.6526 28.194) (width 1) (layer "B.Cu") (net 4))
 (segment (start 90.6526 28.194) (end 115.8748 28.194) (width 1) (layer "B.Cu") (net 4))
 (segment (start 97.0026 60.3504) (end 96.647 60.706) (width 1) (layer "B.Cu") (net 4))
 (segment (start 119.5578 31.877) (end 119.5578 41.148) (width 1) (layer "B.Cu") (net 4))
 (segment (start 93.6244 42.5196) (end 91.821 42.5196) (width 1) (layer "B.Cu") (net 4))
 (segment (start 68.2244 75.5396) (end 70.0532 75.5396) (width 1) (layer "B.Cu") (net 4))
 (segment (start 66.2278 28.717178) (end 66.750978 28.194) (width 1) (layer "B.Cu") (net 4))
 (segment (start 90.2208 40.9194) (end 90.2208 28.6258) (width 1) (layer "B.Cu") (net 4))
 (segment (start 97.8408 75.5904) (end 98.8314 75.5904) (width 1) (layer "B.Cu") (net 4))
 (segment (start 70.0532 75.5396) (end 71.2978 74.295) (width 1) (layer "B.Cu") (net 4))
 (segment (start 63.9572 60.3912) (end 66.2278 60.3912) (width 1) (layer "B.Cu") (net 4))
 (segment (start 91.821 42.5196) (end 90.2208 40.9194) (width 1) (layer "B.Cu") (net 4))
 (segment (start 95.432711 66.670089) (end 96.4692 65.6336) (width 0.4) (layer "F.Cu") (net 25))
 (segment (start 65.298311 66.670089) (end 95.432711 66.670089) (width 0.4) (layer "F.Cu") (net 25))
 (segment (start 96.4692 63.9318) (end 97.5106 62.8904) (width 0.4) (layer "F.Cu") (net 25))
 (segment (start 63.9572 68.0112) (end 65.298311 66.670089) (width 0.4) (layer "F.Cu") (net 25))
 (segment (start 97.5106 62.8904) (end 98.8314 62.8904) (width 0.4) (layer "F.Cu") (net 25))
 (segment (start 96.4692 65.6336) (end 96.4692 63.9318) (width 0.4) (layer "F.Cu") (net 25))
 (segment (start 97.0534 70.5104) (end 98.8314 70.5104) (width 0.4) (layer "F.Cu") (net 28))
 (segment (start 63.9572 65.4712) (end 63.0528 65.4712) (width 0.4) (layer "F.Cu") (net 28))
 (segment (start 63.0528 65.4712) (end 62.2554 66.2686) (width 0.4) (layer "F.Cu") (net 28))
 (segment (start 64.139911 71.709111) (end 95.854689 71.709111) (width 0.4) (layer "F.Cu") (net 28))
 (segment (start 62.2554 66.2686) (end 62.2554 69.8246) (width 0.4) (layer "F.Cu") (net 28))
 (segment (start 95.854689 71.709111) (end 97.0534 70.5104) (width 0.4) (layer "F.Cu") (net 28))
 (segment (start 62.2554 69.8246) (end 64.139911 71.709111) (width 0.4) (layer "F.Cu") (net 28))
 (segment (start 131.318 52.2732) (end 134.366 49.2252) (width 0.4) (layer "F.Cu") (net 13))
 (segment (start 127.1778 52.2732) (end 131.318 52.2732) (width 0.4) (layer "F.Cu") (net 13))
 (segment (start 136.0424 43.18) (end 135.5598 43.6626) (width 0.4) (layer "F.Cu") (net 13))
 (segment (start 101.8032 58.9026) (end 106.684911 54.020889) (width 0.4) (layer "F.Cu") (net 13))
 (segment (start 141.351 43.18) (end 136.0424 43.18) (width 0.4) (layer "F.Cu") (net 13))
 (segment (start 100.2792 73.0504) (end 101.8032 71.5264) (width 0.4) (layer "F.Cu") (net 13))
 (segment (start 101.8032 71.5264) (end 101.8032 58.9026) (width 0.4) (layer "F.Cu") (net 13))
 (segment (start 98.8314 73.0504) (end 100.2792 73.0504) (width 0.4) (layer "F.Cu") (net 13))
 (segment (start 135.5598 43.6626) (end 135.5598 45.1866) (width 0.4) (layer "F.Cu") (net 13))
 (segment (start 141.930289 43.759289) (end 141.351 43.18) (width 0.4) (layer "F.Cu") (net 13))
 (segment (start 141.930289 47.274311) (end 141.930289 43.759289) (width 0.4) (layer "F.Cu") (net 13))
 (segment (start 139.9794 49.2252) (end 141.930289 47.274311) (width 0.4) (layer "F.Cu") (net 13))
 (segment (start 134.366 49.2252) (end 139.9794 49.2252) (width 0.4) (layer "F.Cu") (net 13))
 (segment (start 106.684911 54.020889) (end 125.430111 54.020889) (width 0.4) (layer "F.Cu") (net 13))
 (segment (start 125.430111 54.020889) (end 127.1778 52.2732) (width 0.4) (layer "F.Cu") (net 13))
 (segment (start 98.288178 46.3804) (end 120.2436 46.3804) (width 0.4) (layer "F.Cu") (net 38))
 (segment (start 121.5136 47.6504) (end 124.2314 47.6504) (width 0.4) (layer "F.Cu") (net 38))
 (segment (start 92.1004 50.1396) (end 90.9574 48.9966) (width 0.4) (layer "F.Cu") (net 38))
 (segment (start 120.2436 46.3804) (end 121.5136 47.6504) (width 0.4) (layer "F.Cu") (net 38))
 (segment (start 90.9574 48.9966) (end 90.9574 46.99) (width 0.4) (layer "F.Cu") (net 38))
 (segment (start 98.216889 46.309111) (end 98.288178 46.3804) (width 0.4) (layer "F.Cu") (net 38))
 (segment (start 91.638289 46.309111) (end 98.216889 46.309111) (width 0.4) (layer "F.Cu") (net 38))
 (segment (start 93.6244 50.1396) (end 92.1004 50.1396) (width 0.4) (layer "F.Cu") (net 38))
 (segment (start 90.9574 46.99) (end 91.638289 46.309111) (width 0.4) (layer "F.Cu") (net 38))
 (segment (start 94.965689 48.940889) (end 119.451289 48.940889) (width 0.4) (layer "F.Cu") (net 37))
 (segment (start 120.7008 50.1904) (end 124.2314 50.1904) (width 0.4) (layer "F.Cu") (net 37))
 (segment (start 93.6244 47.5996) (end 94.965689 48.940889) (width 0.4) (layer "F.Cu") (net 37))
 (segment (start 119.451289 48.940889) (end 120.7008 50.1904) (width 0.4) (layer "F.Cu") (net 37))
 (segment (start 130.4798 40.5892) (end 136.4266 34.6424) (width 1) (layer "F.Cu") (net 5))
 (segment (start 130.4798 45.1866) (end 130.4798 40.5892) (width 1) (layer "F.Cu") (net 5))
 (segment (start 136.4266 34.6424) (end 148.3718 34.6424) (width 1) (layer "F.Cu") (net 5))
 (segment (start 160.0708 69.596) (end 160.0708 36.8808) (width 1) (layer "B.Cu") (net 5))
 (segment (start 160.081311 36.870289) (end 160.081311 33.208311) (width 1) (layer "B.Cu") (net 5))
 (segment (start 160.081311 33.208311) (end 159.2326 32.3596) (width 1) (layer "B.Cu") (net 5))
 (segment (start 149.1234 32.3596) (end 148.3718 33.1112) (width 1) (layer "B.Cu") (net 5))
 (segment (start 67.58482 77.1652) (end 122.6566 77.1652) (width 1) (layer "B.Cu") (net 5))
 (segment (start 124.2314 75.5904) (end 154.0764 75.5904) (width 1) (layer "B.Cu") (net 5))
 (segment (start 160.0708 36.8808) (end 160.081311 36.870289) (width 1) (layer "B.Cu") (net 5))
 (segment (start 63.9572 62.9312) (end 66.37478 65.34878) (width 1) (layer "B.Cu") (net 5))
 (segment (start 148.3718 33.1112) (end 148.3718 34.6424) (width 1) (layer "B.Cu") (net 5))
 (segment (start 66.37478 65.34878) (end 66.37478 75.95516) (width 1) (layer "B.Cu") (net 5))
 (segment (start 154.0764 75.5904) (end 160.0708 69.596) (width 1) (layer "B.Cu") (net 5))
 (segment (start 159.2326 32.3596) (end 149.1234 32.3596) (width 1) (layer "B.Cu") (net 5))
 (segment (start 122.6566 77.1652) (end 124.2314 75.5904) (width 1) (layer "B.Cu") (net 5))
 (segment (start 66.37478 75.95516) (end 67.58482 77.1652) (width 1) (layer "B.Cu") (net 5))
 (segment (start 87.4522 56.4896) (end 98.242546 56.4896) (width 0.4) (layer "B.Cu") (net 31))
 (segment (start 122.331311 59.059911) (end 127.262133 59.059911) (width 0.4) (layer "B.Cu") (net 31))
 (segment (start 146.670689 59.421689) (end 147.9202 60.6712) (width 0.4) (layer "B.Cu") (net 31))
 (segment (start 127.623911 59.421689) (end 146.670689 59.421689) (width 0.4) (layer "B.Cu") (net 31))
 (segment (start 127.262133 59.059911) (end 127.623911 59.421689) (width 0.4) (layer "B.Cu") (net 31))
 (segment (start 68.2244 47.5996) (end 78.5622 47.5996) (width 0.4) (layer "B.Cu") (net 31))
 (segment (start 98.242546 56.4896) (end 98.313835 56.560889) (width 0.4) (layer "B.Cu") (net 31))
 (segment (start 119.832289 56.560889) (end 122.331311 59.059911) (width 0.4) (layer "B.Cu") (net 31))
 (segment (start 147.9202 60.6712) (end 152.6036 60.6712) (width 0.4) (layer "B.Cu") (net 31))
 (segment (start 78.5622 47.5996) (end 87.4522 56.4896) (width 0.4) (layer "B.Cu") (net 31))
 (segment (start 98.313835 56.560889) (end 119.832289 56.560889) (width 0.4) (layer "B.Cu") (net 31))
 (segment (start 87.126911 59.009111) (end 98.222057 59.009111) (width 0.4) (layer "B.Cu") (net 30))
 (segment (start 114.599889 59.100889) (end 117.139889 61.640889) (width 0.4) (layer "B.Cu") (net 30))
 (segment (start 127.268311 61.961689) (end 146.086489 61.961689) (width 0.4) (layer "B.Cu") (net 30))
 (segment (start 117.139889 61.640889) (end 126.947511 61.640889) (width 0.4) (layer "B.Cu") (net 30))
 (segment (start 98.313835 59.100889) (end 114.599889 59.100889) (width 0.4) (layer "B.Cu") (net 30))
 (segment (start 147.3548 63.2112) (end 152.6036 63.2112) (width 0.4) (layer "B.Cu") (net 30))
 (segment (start 147.3454 63.2206) (end 147.3548 63.2112) (width 0.4) (layer "B.Cu") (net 30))
 (segment (start 146.086489 61.961689) (end 147.3454 63.2206) (width 0.4) (layer "B.Cu") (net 30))
 (segment (start 126.947511 61.640889) (end 127.268311 61.961689) (width 0.4) (layer "B.Cu") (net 30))
 (segment (start 98.222057 59.009111) (end 98.313835 59.100889) (width 0.4) (layer "B.Cu") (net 30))
 (segment (start 68.2244 50.1396) (end 78.2574 50.1396) (width 0.4) (layer "B.Cu") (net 30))
 (segment (start 78.2574 50.1396) (end 87.126911 59.009111) (width 0.4) (layer "B.Cu") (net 30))
 (segment (start 152.6036 68.2912) (end 157.1896 68.2912) (width 1) (layer "B.Cu") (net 16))
 (segment (start 157.1896 68.2912) (end 157.9372 67.5436) (width 1) (layer "B.Cu") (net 16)))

